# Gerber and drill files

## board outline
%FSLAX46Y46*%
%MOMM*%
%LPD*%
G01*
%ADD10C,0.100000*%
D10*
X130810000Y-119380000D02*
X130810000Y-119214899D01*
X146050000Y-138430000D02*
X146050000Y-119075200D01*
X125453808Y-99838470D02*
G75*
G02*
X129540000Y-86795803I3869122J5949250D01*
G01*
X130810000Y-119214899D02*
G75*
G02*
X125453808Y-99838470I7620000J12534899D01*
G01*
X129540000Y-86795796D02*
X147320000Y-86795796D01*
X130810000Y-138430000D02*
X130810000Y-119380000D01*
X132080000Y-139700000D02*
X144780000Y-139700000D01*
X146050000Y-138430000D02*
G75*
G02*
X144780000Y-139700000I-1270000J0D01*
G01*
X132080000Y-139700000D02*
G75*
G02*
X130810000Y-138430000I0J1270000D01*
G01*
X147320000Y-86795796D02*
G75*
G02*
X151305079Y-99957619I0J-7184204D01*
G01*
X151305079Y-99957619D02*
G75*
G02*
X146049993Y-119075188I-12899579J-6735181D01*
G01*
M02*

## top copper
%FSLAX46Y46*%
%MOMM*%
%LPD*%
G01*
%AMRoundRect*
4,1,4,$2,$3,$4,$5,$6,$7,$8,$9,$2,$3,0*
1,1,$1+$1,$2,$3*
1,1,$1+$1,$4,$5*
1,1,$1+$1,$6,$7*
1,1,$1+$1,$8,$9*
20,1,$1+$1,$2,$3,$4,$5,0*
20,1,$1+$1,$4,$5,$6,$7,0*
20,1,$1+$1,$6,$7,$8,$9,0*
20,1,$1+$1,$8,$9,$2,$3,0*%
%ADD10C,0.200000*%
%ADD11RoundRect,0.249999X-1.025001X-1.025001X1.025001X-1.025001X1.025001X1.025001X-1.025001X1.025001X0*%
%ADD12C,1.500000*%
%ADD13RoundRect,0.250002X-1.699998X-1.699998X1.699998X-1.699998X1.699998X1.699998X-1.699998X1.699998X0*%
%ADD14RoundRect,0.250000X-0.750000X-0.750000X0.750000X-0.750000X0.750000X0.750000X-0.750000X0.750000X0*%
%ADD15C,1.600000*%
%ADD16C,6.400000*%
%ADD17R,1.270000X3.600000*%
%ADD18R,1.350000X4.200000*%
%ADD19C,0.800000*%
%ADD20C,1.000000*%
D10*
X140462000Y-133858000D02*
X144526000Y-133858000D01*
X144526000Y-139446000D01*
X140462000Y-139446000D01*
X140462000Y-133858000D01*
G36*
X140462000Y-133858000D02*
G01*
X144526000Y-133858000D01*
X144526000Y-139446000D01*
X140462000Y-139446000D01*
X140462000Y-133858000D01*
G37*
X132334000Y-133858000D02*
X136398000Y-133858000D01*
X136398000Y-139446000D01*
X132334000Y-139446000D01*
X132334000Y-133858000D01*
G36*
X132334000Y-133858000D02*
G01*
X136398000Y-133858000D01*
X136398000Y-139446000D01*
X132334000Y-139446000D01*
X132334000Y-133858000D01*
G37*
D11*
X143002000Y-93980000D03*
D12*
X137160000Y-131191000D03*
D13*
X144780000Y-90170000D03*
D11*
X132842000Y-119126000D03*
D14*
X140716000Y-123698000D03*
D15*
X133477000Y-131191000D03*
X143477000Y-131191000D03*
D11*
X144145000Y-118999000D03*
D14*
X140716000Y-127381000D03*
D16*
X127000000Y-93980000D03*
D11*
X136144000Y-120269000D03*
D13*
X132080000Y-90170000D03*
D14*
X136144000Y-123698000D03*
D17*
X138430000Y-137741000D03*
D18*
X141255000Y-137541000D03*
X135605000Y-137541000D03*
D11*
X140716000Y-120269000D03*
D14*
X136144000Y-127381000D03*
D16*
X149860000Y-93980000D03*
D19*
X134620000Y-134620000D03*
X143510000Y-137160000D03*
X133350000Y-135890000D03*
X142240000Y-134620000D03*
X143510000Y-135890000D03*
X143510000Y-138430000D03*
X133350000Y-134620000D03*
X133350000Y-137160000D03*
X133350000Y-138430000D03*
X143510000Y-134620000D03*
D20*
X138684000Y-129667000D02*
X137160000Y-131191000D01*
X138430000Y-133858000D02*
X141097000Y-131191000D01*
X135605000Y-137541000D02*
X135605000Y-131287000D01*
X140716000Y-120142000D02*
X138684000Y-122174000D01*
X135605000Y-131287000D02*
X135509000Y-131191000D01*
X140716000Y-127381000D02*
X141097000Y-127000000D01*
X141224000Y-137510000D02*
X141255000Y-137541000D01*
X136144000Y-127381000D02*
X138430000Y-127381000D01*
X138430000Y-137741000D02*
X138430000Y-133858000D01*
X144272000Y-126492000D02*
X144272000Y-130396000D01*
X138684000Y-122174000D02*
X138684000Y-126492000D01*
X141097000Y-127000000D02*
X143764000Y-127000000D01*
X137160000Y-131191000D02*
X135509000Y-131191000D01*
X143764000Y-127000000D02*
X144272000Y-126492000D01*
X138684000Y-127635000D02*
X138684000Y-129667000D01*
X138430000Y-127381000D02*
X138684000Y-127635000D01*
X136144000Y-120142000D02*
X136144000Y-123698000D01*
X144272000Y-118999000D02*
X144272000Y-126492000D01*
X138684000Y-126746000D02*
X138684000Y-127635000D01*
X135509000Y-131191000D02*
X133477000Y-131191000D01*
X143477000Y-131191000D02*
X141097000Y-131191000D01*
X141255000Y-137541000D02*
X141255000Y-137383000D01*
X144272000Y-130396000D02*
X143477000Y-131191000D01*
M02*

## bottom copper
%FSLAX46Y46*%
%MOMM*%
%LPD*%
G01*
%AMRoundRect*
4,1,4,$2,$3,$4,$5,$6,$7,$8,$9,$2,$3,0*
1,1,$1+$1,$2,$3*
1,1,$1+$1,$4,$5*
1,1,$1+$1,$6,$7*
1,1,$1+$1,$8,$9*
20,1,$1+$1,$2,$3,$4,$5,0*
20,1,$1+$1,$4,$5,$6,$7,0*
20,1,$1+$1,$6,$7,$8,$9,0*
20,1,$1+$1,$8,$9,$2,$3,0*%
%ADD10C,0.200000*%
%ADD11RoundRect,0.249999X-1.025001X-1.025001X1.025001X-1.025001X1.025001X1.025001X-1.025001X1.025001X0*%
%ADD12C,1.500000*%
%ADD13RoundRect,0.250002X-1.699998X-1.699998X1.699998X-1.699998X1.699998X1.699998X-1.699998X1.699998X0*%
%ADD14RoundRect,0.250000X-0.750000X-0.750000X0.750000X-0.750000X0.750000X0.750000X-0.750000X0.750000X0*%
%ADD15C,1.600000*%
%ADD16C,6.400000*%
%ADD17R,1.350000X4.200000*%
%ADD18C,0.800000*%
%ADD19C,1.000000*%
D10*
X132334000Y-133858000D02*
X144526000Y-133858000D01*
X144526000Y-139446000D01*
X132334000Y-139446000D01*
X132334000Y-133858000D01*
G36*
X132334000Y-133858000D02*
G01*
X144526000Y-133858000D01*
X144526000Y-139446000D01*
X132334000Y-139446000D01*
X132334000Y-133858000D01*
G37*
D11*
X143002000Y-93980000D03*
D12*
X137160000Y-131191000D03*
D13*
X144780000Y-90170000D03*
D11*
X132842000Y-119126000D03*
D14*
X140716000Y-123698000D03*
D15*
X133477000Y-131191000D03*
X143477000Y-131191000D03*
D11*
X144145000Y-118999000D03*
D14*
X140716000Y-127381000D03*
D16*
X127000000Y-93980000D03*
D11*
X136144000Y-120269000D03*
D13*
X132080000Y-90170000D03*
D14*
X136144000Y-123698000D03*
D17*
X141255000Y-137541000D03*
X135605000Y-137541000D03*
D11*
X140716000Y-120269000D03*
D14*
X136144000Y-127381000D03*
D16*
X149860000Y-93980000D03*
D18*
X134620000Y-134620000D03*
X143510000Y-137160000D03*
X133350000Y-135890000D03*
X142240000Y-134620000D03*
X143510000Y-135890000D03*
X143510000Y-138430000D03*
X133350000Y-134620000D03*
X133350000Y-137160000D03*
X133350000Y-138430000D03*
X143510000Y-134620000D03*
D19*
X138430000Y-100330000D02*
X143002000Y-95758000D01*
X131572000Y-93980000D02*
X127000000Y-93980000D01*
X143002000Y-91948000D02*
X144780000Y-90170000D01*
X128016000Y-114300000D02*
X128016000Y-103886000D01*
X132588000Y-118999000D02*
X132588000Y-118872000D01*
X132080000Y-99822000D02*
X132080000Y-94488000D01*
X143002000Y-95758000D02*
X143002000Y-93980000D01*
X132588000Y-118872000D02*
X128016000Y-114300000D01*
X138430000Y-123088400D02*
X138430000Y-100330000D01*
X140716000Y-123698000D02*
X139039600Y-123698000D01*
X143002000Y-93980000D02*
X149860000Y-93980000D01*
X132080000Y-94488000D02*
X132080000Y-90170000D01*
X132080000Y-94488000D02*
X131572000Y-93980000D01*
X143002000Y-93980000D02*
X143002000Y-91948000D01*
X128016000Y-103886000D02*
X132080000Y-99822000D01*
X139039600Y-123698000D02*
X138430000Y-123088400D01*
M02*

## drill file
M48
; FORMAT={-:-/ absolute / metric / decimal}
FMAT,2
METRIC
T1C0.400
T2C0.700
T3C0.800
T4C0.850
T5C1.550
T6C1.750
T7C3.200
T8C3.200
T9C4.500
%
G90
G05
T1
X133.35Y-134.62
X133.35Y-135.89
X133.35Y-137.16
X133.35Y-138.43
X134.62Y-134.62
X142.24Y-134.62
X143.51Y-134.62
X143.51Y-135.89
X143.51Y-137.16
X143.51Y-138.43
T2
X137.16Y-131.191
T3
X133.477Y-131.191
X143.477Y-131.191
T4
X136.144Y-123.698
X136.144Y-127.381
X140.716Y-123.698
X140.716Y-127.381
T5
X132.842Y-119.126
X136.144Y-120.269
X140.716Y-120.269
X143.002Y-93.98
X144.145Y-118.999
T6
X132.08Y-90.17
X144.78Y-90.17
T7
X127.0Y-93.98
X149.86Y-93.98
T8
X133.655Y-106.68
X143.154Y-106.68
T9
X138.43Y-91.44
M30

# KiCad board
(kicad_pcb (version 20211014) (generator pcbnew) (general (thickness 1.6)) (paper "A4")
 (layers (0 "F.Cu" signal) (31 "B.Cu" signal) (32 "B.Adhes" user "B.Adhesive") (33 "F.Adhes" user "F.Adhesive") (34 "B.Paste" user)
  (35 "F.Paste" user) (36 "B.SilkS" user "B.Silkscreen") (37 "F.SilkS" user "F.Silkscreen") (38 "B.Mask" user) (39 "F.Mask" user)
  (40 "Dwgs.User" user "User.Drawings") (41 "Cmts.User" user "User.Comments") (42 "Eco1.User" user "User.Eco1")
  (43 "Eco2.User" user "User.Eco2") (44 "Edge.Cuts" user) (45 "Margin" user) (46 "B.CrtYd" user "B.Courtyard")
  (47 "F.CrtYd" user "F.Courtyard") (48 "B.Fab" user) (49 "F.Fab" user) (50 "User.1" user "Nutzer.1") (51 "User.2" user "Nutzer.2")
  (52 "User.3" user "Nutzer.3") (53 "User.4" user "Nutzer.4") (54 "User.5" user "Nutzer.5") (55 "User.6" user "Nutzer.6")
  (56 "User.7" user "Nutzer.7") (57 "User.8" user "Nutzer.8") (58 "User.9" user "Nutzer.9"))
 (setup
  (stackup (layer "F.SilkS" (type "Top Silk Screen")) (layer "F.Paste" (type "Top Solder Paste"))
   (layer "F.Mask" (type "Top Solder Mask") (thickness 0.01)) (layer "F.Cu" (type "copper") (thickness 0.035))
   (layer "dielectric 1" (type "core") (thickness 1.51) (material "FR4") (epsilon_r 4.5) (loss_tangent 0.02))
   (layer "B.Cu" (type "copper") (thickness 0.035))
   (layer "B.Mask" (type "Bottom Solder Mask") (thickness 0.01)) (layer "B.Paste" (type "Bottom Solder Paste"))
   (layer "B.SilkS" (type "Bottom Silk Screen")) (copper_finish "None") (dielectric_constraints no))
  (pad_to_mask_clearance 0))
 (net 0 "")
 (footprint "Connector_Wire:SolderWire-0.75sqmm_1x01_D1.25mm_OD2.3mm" (layer "F.Cu") (at 143.002 93.98)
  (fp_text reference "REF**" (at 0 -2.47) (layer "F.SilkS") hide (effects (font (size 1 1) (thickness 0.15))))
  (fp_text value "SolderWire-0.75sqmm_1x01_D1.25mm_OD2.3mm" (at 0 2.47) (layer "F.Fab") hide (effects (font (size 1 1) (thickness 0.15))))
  (pad "1" thru_hole roundrect (at 0 0) (size 2.55 2.55) (drill 1.55) (layers *.Cu *.Mask) (roundrect_rratio 0.098039)))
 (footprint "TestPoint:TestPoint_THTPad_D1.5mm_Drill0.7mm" (layer "F.Cu") (at 137.16 131.191)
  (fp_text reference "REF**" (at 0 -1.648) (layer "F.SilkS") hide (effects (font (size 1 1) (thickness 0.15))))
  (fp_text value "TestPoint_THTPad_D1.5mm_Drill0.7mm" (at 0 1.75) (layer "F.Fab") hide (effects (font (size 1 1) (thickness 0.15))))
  (pad "1" thru_hole circle (at 0 0) (size 1.5 1.5) (drill 0.7) (layers *.Cu *.Mask)))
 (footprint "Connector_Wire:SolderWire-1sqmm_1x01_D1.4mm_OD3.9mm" (layer "F.Cu") (at 144.78 90.17)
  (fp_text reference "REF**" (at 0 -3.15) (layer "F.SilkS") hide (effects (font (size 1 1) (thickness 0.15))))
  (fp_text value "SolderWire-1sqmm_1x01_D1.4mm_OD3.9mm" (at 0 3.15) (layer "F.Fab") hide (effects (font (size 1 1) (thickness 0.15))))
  (pad "1" thru_hole roundrect (at 0 0) (size 3.9 3.9) (drill 1.75) (layers *.Cu *.Mask) (roundrect_rratio 0.064103)))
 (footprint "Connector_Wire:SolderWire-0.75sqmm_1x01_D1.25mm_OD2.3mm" (layer "F.Cu") (at 132.842 119.126)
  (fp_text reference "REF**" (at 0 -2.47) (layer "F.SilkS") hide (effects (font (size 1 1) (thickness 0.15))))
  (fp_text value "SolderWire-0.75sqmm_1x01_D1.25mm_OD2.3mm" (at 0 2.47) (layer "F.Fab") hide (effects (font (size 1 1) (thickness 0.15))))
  (pad "1" thru_hole roundrect (at 0 0) (size 2.55 2.55) (drill 1.55) (layers *.Cu *.Mask) (roundrect_rratio 0.098039)))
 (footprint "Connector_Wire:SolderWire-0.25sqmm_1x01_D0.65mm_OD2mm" (layer "F.Cu") (at 140.716 123.698)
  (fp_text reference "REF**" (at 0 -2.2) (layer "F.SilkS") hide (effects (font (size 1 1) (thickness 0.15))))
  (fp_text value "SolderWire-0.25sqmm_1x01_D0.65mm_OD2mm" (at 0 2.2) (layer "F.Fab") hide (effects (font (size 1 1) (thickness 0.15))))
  (pad "1" thru_hole roundrect (at 0 0) (size 2 2) (drill 0.85) (layers *.Cu *.Mask) (roundrect_rratio 0.125)))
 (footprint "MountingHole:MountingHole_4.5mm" (layer "F.Cu") (at 138.43 91.44)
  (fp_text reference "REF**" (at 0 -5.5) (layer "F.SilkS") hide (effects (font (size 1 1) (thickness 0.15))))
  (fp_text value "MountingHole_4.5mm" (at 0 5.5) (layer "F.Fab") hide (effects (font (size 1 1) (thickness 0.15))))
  (pad "" np_thru_hole circle (at 0 0) (size 4.5 4.5) (drill 4.5) (layers *.Cu *.Mask)))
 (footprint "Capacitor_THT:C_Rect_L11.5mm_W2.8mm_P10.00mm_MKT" (layer "F.Cu") (at 133.477 131.191)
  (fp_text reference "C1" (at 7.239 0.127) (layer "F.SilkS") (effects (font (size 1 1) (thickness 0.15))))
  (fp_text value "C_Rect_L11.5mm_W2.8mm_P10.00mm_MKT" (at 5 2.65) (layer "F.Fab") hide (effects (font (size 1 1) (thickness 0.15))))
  (pad "1" thru_hole circle (at 0 0) (size 1.6 1.6) (drill 0.8) (layers *.Cu *.Mask))
  (pad "2" thru_hole circle (at 10 0) (size 1.6 1.6) (drill 0.8) (layers *.Cu *.Mask)))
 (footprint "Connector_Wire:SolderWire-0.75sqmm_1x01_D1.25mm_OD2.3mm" (layer "F.Cu") (at 144.145 118.999)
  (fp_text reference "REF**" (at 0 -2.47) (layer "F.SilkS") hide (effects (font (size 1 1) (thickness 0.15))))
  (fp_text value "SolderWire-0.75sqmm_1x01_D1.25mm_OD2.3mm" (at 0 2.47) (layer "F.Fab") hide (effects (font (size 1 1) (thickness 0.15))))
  (pad "1" thru_hole roundrect (at 0 0) (size 2.55 2.55) (drill 1.55) (layers *.Cu *.Mask) (roundrect_rratio 0.098039)))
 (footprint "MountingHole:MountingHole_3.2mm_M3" (layer "F.Cu") (at 143.1544 106.68)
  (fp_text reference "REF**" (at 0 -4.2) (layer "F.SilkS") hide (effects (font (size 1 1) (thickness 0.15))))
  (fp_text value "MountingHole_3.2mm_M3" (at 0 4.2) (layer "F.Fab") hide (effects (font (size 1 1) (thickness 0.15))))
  (pad "" np_thru_hole circle (at 0 0) (size 3.2 3.2) (drill 3.2) (layers *.Cu *.Mask)))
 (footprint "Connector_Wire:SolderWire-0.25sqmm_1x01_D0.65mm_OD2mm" (layer "F.Cu") (at 140.716 127.381)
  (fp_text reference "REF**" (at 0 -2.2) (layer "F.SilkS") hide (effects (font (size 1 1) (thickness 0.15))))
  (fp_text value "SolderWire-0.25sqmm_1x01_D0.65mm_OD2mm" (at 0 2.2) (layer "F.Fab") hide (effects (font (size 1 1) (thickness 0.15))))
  (pad "1" thru_hole roundrect (at 0 0) (size 2 2) (drill 0.85) (layers *.Cu *.Mask) (roundrect_rratio 0.125)))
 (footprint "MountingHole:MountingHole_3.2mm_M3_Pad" (layer "F.Cu") (at 127 93.98)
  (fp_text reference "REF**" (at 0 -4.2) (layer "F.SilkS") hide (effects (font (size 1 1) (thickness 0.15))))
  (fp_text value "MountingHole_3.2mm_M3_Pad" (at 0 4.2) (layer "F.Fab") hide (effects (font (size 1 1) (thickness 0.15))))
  (pad "1" thru_hole circle (at 0 0) (size 6.4 6.4) (drill 3.2) (layers *.Cu *.Mask)))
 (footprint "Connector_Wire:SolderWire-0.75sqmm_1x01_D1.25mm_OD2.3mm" (layer "F.Cu") (at 136.144 120.269)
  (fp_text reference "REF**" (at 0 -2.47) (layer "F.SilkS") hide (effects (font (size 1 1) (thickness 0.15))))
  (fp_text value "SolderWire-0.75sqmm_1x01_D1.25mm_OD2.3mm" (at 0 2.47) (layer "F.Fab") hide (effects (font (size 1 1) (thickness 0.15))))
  (pad "1" thru_hole roundrect (at 0 0) (size 2.55 2.55) (drill 1.55) (layers *.Cu *.Mask) (roundrect_rratio 0.098039)))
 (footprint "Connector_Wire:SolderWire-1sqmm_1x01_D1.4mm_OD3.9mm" (layer "F.Cu") (at 132.08 90.17)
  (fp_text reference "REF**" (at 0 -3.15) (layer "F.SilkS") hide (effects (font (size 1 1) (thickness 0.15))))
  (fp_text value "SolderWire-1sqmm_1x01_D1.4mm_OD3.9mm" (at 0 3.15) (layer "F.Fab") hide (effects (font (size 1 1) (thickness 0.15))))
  (pad "1" thru_hole roundrect (at 0 0) (size 3.9 3.9) (drill 1.75) (layers *.Cu *.Mask) (roundrect_rratio 0.064103)))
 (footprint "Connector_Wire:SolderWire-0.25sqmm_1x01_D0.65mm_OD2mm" (layer "F.Cu") (at 136.144 123.698)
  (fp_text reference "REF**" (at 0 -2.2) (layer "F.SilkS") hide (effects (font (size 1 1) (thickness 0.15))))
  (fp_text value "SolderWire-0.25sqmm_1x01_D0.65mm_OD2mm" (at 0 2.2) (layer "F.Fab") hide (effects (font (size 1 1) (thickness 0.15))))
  (pad "1" thru_hole roundrect (at 0 0) (size 2 2) (drill 0.85) (layers *.Cu *.Mask) (roundrect_rratio 0.125)))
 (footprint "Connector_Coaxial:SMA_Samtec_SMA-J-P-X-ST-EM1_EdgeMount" (layer "F.Cu") (at 138.43 137.541)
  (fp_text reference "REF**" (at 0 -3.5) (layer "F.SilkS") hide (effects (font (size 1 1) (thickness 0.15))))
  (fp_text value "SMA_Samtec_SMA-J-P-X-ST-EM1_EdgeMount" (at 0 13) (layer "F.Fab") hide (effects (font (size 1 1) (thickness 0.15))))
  (pad "1" smd rect (at 0 0.2) (size 1.27 3.6) (layers "F.Cu" "F.Paste" "F.Mask"))
  (pad "2" smd rect (at 2.825 0) (size 1.35 4.2) (layers "F.Cu" "F.Paste" "F.Mask"))
  (pad "2" smd rect (at 2.825 0) (size 1.35 4.2) (layers "B.Cu" "B.Paste" "B.Mask"))
  (pad "2" smd rect (at -2.825 0) (size 1.35 4.2) (layers "B.Cu" "B.Paste" "B.Mask"))
  (pad "2" smd rect (at -2.825 0) (size 1.35 4.2) (layers "F.Cu" "F.Paste" "F.Mask")))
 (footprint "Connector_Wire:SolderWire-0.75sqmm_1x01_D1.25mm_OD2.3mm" (layer "F.Cu") (at 140.716 120.269)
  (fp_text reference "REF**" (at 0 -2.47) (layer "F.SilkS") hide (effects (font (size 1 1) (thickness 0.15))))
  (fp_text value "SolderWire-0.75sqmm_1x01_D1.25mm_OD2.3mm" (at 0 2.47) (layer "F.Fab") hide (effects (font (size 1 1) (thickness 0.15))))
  (pad "1" thru_hole roundrect (at 0 0) (size 2.55 2.55) (drill 1.55) (layers *.Cu *.Mask) (roundrect_rratio 0.098039)))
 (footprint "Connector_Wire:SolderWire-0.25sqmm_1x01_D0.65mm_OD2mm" (layer "F.Cu") (at 136.144 127.381)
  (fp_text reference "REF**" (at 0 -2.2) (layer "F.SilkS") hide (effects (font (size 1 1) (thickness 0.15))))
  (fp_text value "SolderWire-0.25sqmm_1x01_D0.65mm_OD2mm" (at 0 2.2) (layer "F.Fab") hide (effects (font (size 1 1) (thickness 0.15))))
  (pad "1" thru_hole roundrect (at 0 0) (size 2 2) (drill 0.85) (layers *.Cu *.Mask) (roundrect_rratio 0.125)))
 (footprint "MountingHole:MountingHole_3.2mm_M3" (layer "F.Cu") (at 133.6548 106.68)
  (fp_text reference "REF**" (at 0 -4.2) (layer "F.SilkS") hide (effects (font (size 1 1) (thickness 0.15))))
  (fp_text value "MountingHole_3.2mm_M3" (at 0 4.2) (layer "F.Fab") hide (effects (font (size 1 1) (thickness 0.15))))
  (pad "" np_thru_hole circle (at 0 0) (size 3.2 3.2) (drill 3.2) (layers *.Cu *.Mask)))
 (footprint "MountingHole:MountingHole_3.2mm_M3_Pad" (layer "F.Cu") (at 149.86 93.98)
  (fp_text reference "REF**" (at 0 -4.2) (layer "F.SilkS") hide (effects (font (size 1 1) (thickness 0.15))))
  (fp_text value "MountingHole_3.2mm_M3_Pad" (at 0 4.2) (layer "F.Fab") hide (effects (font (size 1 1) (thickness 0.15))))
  (pad "1" thru_hole circle (at 0 0) (size 6.4 6.4) (drill 3.2) (layers *.Cu *.Mask)))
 (gr_rect (start 144.526 133.858) (end 140.462 139.446) (layer "F.Cu") (width 0.2) (fill solid))
 (gr_rect (start 132.334 133.858) (end 136.398 139.446) (layer "F.Cu") (width 0.2) (fill solid))
 (gr_rect (start 132.334 133.858) (end 144.526 139.446) (layer "B.Cu") (width 0.2) (fill solid))
 (gr_line (start 130.81 119.38) (end 130.81 119.214899) (layer "Edge.Cuts") (width 0.1))
 (gr_line (start 146.05 138.43) (end 146.05 119.0752) (layer "Edge.Cuts") (width 0.1))
 (gr_arc (start 125.453808 99.83847) (mid 122.550769 91.767538) (end 129.54 86.795796) (layer "Edge.Cuts") (width 0.1))
 (gr_arc (start 130.81 119.214899) (mid 124.290966 110.588428) (end 125.453808 99.83847) (layer "Edge.Cuts") (width 0.1))
 (gr_line (start 129.54 86.795796) (end 147.32 86.795796) (layer "Edge.Cuts") (width 0.1))
 (gr_line (start 130.81 138.43) (end 130.81 119.38) (layer "Edge.Cuts") (width 0.1))
 (gr_line (start 132.08 139.7) (end 144.78 139.7) (layer "Edge.Cuts") (width 0.1))
 (gr_arc (start 146.05 138.43) (mid 145.678026 139.328026) (end 144.78 139.7) (layer "Edge.Cuts") (width 0.1))
 (gr_arc (start 132.08 139.7) (mid 131.181974 139.328026) (end 130.81 138.43) (layer "Edge.Cuts") (width 0.1))
 (gr_arc (start 147.32 86.795796) (mid 154.195942 91.898132) (end 151.305079 99.957619) (layer "Edge.Cuts") (width 0.1))
 (gr_arc (start 151.305079 99.957619) (mid 152.437075 110.549838) (end 146.05 119.0752) (layer "Edge.Cuts") (width 0.1))
 (segment (start 138.684 129.667) (end 137.16 131.191) (width 1) (layer "F.Cu") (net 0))
 (segment (start 138.43 133.858) (end 141.097 131.191) (width 1) (layer "F.Cu") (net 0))
 (segment (start 135.605 137.541) (end 135.605 131.287) (width 1) (layer "F.Cu") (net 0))
 (segment (start 140.716 120.142) (end 138.684 122.174) (width 1) (layer "F.Cu") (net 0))
 (segment (start 135.605 131.287) (end 135.509 131.191) (width 1) (layer "F.Cu") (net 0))
 (segment (start 140.716 127.381) (end 141.097 127) (width 1) (layer "F.Cu") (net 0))
 (segment (start 141.224 137.51) (end 141.255 137.541) (width 1) (layer "F.Cu") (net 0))
 (segment (start 136.144 127.381) (end 138.43 127.381) (width 1) (layer "F.Cu") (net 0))
 (segment (start 138.43 137.741) (end 138.43 133.858) (width 1) (layer "F.Cu") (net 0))
 (segment (start 144.272 126.492) (end 144.272 130.396) (width 1) (layer "F.Cu") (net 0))
 (segment (start 138.684 122.174) (end 138.684 126.492) (width 1) (layer "F.Cu") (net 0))
 (segment (start 141.097 127) (end 143.764 127) (width 1) (layer "F.Cu") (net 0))
 (segment (start 137.16 131.191) (end 135.509 131.191) (width 1) (layer "F.Cu") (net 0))
 (segment (start 143.764 127) (end 144.272 126.492) (width 1) (layer "F.Cu") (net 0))
 (segment (start 138.684 127.635) (end 138.684 129.667) (width 1) (layer "F.Cu") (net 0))
 (segment (start 138.43 127.381) (end 138.684 127.635) (width 1) (layer "F.Cu") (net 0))
 (segment (start 136.144 120.142) (end 136.144 123.698) (width 1) (layer "F.Cu") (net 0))
 (segment (start 144.272 118.999) (end 144.272 126.492) (width 1) (layer "F.Cu") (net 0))
 (segment (start 138.684 126.746) (end 138.684 127.635) (width 1) (layer "F.Cu") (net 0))
 (segment (start 135.509 131.191) (end 133.477 131.191) (width 1) (layer "F.Cu") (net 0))
 (segment (start 143.477 131.191) (end 141.097 131.191) (width 1) (layer "F.Cu") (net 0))
 (segment (start 141.255 137.541) (end 141.255 137.383) (width 1) (layer "F.Cu") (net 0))
 (segment (start 144.272 130.396) (end 143.477 131.191) (width 1) (layer "F.Cu") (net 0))
 (via (at 134.62 134.62) (size 0.8) (drill 0.4) (layers "F.Cu" "B.Cu") (free) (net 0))
 (via (at 143.51 137.16) (size 0.8) (drill 0.4) (layers "F.Cu" "B.Cu") (free) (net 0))
 (via (at 133.35 135.89) (size 0.8) (drill 0.4) (layers "F.Cu" "B.Cu") (free) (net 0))
 (via (at 142.24 134.62) (size 0.8) (drill 0.4) (layers "F.Cu" "B.Cu") (free) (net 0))
 (via (at 143.51 135.89) (size 0.8) (drill 0.4) (layers "F.Cu" "B.Cu") (free) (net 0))
 (via (at 143.51 138.43) (size 0.8) (drill 0.4) (layers "F.Cu" "B.Cu") (free) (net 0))
 (via (at 133.35 134.62) (size 0.8) (drill 0.4) (layers "F.Cu" "B.Cu") (free) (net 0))
 (via (at 133.35 137.16) (size 0.8) (drill 0.4) (layers "F.Cu" "B.Cu") (free) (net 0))
 (via (at 133.35 138.43) (size 0.8) (drill 0.4) (layers "F.Cu" "B.Cu") (free) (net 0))
 (via (at 143.51 134.62) (size 0.8) (drill 0.4) (layers "F.Cu" "B.Cu") (free) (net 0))
 (segment (start 138.43 100.33) (end 143.002 95.758) (width 1) (layer "B.Cu") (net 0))
 (segment (start 131.572 93.98) (end 127 93.98) (width 1) (layer "B.Cu") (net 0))
 (segment (start 143.002 91.948) (end 144.78 90.17) (width 1) (layer "B.Cu") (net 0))
 (segment (start 128.016 114.3) (end 128.016 103.886) (width 1) (layer "B.Cu") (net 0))
 (segment (start 132.588 118.999) (end 132.588 118.872) (width 1) (layer "B.Cu") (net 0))
 (segment (start 132.08 99.822) (end 132.08 94.488) (width 1) (layer "B.Cu") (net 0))
 (segment (start 143.002 95.758) (end 143.002 93.98) (width 1) (layer "B.Cu") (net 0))
 (segment (start 132.588 118.872) (end 128.016 114.3) (width 1) (layer "B.Cu") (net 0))
 (segment (start 138.43 123.0884) (end 138.43 100.33) (width 1) (layer "B.Cu") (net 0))
 (segment (start 140.716 123.698) (end 139.0396 123.698) (width 1) (layer "B.Cu") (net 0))
 (segment (start 143.002 93.98) (end 149.86 93.98) (width 1) (layer "B.Cu") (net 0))
 (segment (start 132.08 94.488) (end 132.08 90.17) (width 1) (layer "B.Cu") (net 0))
 (segment (start 132.08 94.488) (end 131.572 93.98) (width 1) (layer "B.Cu") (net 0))
 (segment (start 143.002 93.98) (end 143.002 91.948) (width 1) (layer "B.Cu") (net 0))
 (segment (start 128.016 103.886) (end 132.08 99.822) (width 1) (layer "B.Cu") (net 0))
 (segment (start 139.0396 123.698) (end 138.43 123.0884) (width 1) (layer "B.Cu") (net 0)))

